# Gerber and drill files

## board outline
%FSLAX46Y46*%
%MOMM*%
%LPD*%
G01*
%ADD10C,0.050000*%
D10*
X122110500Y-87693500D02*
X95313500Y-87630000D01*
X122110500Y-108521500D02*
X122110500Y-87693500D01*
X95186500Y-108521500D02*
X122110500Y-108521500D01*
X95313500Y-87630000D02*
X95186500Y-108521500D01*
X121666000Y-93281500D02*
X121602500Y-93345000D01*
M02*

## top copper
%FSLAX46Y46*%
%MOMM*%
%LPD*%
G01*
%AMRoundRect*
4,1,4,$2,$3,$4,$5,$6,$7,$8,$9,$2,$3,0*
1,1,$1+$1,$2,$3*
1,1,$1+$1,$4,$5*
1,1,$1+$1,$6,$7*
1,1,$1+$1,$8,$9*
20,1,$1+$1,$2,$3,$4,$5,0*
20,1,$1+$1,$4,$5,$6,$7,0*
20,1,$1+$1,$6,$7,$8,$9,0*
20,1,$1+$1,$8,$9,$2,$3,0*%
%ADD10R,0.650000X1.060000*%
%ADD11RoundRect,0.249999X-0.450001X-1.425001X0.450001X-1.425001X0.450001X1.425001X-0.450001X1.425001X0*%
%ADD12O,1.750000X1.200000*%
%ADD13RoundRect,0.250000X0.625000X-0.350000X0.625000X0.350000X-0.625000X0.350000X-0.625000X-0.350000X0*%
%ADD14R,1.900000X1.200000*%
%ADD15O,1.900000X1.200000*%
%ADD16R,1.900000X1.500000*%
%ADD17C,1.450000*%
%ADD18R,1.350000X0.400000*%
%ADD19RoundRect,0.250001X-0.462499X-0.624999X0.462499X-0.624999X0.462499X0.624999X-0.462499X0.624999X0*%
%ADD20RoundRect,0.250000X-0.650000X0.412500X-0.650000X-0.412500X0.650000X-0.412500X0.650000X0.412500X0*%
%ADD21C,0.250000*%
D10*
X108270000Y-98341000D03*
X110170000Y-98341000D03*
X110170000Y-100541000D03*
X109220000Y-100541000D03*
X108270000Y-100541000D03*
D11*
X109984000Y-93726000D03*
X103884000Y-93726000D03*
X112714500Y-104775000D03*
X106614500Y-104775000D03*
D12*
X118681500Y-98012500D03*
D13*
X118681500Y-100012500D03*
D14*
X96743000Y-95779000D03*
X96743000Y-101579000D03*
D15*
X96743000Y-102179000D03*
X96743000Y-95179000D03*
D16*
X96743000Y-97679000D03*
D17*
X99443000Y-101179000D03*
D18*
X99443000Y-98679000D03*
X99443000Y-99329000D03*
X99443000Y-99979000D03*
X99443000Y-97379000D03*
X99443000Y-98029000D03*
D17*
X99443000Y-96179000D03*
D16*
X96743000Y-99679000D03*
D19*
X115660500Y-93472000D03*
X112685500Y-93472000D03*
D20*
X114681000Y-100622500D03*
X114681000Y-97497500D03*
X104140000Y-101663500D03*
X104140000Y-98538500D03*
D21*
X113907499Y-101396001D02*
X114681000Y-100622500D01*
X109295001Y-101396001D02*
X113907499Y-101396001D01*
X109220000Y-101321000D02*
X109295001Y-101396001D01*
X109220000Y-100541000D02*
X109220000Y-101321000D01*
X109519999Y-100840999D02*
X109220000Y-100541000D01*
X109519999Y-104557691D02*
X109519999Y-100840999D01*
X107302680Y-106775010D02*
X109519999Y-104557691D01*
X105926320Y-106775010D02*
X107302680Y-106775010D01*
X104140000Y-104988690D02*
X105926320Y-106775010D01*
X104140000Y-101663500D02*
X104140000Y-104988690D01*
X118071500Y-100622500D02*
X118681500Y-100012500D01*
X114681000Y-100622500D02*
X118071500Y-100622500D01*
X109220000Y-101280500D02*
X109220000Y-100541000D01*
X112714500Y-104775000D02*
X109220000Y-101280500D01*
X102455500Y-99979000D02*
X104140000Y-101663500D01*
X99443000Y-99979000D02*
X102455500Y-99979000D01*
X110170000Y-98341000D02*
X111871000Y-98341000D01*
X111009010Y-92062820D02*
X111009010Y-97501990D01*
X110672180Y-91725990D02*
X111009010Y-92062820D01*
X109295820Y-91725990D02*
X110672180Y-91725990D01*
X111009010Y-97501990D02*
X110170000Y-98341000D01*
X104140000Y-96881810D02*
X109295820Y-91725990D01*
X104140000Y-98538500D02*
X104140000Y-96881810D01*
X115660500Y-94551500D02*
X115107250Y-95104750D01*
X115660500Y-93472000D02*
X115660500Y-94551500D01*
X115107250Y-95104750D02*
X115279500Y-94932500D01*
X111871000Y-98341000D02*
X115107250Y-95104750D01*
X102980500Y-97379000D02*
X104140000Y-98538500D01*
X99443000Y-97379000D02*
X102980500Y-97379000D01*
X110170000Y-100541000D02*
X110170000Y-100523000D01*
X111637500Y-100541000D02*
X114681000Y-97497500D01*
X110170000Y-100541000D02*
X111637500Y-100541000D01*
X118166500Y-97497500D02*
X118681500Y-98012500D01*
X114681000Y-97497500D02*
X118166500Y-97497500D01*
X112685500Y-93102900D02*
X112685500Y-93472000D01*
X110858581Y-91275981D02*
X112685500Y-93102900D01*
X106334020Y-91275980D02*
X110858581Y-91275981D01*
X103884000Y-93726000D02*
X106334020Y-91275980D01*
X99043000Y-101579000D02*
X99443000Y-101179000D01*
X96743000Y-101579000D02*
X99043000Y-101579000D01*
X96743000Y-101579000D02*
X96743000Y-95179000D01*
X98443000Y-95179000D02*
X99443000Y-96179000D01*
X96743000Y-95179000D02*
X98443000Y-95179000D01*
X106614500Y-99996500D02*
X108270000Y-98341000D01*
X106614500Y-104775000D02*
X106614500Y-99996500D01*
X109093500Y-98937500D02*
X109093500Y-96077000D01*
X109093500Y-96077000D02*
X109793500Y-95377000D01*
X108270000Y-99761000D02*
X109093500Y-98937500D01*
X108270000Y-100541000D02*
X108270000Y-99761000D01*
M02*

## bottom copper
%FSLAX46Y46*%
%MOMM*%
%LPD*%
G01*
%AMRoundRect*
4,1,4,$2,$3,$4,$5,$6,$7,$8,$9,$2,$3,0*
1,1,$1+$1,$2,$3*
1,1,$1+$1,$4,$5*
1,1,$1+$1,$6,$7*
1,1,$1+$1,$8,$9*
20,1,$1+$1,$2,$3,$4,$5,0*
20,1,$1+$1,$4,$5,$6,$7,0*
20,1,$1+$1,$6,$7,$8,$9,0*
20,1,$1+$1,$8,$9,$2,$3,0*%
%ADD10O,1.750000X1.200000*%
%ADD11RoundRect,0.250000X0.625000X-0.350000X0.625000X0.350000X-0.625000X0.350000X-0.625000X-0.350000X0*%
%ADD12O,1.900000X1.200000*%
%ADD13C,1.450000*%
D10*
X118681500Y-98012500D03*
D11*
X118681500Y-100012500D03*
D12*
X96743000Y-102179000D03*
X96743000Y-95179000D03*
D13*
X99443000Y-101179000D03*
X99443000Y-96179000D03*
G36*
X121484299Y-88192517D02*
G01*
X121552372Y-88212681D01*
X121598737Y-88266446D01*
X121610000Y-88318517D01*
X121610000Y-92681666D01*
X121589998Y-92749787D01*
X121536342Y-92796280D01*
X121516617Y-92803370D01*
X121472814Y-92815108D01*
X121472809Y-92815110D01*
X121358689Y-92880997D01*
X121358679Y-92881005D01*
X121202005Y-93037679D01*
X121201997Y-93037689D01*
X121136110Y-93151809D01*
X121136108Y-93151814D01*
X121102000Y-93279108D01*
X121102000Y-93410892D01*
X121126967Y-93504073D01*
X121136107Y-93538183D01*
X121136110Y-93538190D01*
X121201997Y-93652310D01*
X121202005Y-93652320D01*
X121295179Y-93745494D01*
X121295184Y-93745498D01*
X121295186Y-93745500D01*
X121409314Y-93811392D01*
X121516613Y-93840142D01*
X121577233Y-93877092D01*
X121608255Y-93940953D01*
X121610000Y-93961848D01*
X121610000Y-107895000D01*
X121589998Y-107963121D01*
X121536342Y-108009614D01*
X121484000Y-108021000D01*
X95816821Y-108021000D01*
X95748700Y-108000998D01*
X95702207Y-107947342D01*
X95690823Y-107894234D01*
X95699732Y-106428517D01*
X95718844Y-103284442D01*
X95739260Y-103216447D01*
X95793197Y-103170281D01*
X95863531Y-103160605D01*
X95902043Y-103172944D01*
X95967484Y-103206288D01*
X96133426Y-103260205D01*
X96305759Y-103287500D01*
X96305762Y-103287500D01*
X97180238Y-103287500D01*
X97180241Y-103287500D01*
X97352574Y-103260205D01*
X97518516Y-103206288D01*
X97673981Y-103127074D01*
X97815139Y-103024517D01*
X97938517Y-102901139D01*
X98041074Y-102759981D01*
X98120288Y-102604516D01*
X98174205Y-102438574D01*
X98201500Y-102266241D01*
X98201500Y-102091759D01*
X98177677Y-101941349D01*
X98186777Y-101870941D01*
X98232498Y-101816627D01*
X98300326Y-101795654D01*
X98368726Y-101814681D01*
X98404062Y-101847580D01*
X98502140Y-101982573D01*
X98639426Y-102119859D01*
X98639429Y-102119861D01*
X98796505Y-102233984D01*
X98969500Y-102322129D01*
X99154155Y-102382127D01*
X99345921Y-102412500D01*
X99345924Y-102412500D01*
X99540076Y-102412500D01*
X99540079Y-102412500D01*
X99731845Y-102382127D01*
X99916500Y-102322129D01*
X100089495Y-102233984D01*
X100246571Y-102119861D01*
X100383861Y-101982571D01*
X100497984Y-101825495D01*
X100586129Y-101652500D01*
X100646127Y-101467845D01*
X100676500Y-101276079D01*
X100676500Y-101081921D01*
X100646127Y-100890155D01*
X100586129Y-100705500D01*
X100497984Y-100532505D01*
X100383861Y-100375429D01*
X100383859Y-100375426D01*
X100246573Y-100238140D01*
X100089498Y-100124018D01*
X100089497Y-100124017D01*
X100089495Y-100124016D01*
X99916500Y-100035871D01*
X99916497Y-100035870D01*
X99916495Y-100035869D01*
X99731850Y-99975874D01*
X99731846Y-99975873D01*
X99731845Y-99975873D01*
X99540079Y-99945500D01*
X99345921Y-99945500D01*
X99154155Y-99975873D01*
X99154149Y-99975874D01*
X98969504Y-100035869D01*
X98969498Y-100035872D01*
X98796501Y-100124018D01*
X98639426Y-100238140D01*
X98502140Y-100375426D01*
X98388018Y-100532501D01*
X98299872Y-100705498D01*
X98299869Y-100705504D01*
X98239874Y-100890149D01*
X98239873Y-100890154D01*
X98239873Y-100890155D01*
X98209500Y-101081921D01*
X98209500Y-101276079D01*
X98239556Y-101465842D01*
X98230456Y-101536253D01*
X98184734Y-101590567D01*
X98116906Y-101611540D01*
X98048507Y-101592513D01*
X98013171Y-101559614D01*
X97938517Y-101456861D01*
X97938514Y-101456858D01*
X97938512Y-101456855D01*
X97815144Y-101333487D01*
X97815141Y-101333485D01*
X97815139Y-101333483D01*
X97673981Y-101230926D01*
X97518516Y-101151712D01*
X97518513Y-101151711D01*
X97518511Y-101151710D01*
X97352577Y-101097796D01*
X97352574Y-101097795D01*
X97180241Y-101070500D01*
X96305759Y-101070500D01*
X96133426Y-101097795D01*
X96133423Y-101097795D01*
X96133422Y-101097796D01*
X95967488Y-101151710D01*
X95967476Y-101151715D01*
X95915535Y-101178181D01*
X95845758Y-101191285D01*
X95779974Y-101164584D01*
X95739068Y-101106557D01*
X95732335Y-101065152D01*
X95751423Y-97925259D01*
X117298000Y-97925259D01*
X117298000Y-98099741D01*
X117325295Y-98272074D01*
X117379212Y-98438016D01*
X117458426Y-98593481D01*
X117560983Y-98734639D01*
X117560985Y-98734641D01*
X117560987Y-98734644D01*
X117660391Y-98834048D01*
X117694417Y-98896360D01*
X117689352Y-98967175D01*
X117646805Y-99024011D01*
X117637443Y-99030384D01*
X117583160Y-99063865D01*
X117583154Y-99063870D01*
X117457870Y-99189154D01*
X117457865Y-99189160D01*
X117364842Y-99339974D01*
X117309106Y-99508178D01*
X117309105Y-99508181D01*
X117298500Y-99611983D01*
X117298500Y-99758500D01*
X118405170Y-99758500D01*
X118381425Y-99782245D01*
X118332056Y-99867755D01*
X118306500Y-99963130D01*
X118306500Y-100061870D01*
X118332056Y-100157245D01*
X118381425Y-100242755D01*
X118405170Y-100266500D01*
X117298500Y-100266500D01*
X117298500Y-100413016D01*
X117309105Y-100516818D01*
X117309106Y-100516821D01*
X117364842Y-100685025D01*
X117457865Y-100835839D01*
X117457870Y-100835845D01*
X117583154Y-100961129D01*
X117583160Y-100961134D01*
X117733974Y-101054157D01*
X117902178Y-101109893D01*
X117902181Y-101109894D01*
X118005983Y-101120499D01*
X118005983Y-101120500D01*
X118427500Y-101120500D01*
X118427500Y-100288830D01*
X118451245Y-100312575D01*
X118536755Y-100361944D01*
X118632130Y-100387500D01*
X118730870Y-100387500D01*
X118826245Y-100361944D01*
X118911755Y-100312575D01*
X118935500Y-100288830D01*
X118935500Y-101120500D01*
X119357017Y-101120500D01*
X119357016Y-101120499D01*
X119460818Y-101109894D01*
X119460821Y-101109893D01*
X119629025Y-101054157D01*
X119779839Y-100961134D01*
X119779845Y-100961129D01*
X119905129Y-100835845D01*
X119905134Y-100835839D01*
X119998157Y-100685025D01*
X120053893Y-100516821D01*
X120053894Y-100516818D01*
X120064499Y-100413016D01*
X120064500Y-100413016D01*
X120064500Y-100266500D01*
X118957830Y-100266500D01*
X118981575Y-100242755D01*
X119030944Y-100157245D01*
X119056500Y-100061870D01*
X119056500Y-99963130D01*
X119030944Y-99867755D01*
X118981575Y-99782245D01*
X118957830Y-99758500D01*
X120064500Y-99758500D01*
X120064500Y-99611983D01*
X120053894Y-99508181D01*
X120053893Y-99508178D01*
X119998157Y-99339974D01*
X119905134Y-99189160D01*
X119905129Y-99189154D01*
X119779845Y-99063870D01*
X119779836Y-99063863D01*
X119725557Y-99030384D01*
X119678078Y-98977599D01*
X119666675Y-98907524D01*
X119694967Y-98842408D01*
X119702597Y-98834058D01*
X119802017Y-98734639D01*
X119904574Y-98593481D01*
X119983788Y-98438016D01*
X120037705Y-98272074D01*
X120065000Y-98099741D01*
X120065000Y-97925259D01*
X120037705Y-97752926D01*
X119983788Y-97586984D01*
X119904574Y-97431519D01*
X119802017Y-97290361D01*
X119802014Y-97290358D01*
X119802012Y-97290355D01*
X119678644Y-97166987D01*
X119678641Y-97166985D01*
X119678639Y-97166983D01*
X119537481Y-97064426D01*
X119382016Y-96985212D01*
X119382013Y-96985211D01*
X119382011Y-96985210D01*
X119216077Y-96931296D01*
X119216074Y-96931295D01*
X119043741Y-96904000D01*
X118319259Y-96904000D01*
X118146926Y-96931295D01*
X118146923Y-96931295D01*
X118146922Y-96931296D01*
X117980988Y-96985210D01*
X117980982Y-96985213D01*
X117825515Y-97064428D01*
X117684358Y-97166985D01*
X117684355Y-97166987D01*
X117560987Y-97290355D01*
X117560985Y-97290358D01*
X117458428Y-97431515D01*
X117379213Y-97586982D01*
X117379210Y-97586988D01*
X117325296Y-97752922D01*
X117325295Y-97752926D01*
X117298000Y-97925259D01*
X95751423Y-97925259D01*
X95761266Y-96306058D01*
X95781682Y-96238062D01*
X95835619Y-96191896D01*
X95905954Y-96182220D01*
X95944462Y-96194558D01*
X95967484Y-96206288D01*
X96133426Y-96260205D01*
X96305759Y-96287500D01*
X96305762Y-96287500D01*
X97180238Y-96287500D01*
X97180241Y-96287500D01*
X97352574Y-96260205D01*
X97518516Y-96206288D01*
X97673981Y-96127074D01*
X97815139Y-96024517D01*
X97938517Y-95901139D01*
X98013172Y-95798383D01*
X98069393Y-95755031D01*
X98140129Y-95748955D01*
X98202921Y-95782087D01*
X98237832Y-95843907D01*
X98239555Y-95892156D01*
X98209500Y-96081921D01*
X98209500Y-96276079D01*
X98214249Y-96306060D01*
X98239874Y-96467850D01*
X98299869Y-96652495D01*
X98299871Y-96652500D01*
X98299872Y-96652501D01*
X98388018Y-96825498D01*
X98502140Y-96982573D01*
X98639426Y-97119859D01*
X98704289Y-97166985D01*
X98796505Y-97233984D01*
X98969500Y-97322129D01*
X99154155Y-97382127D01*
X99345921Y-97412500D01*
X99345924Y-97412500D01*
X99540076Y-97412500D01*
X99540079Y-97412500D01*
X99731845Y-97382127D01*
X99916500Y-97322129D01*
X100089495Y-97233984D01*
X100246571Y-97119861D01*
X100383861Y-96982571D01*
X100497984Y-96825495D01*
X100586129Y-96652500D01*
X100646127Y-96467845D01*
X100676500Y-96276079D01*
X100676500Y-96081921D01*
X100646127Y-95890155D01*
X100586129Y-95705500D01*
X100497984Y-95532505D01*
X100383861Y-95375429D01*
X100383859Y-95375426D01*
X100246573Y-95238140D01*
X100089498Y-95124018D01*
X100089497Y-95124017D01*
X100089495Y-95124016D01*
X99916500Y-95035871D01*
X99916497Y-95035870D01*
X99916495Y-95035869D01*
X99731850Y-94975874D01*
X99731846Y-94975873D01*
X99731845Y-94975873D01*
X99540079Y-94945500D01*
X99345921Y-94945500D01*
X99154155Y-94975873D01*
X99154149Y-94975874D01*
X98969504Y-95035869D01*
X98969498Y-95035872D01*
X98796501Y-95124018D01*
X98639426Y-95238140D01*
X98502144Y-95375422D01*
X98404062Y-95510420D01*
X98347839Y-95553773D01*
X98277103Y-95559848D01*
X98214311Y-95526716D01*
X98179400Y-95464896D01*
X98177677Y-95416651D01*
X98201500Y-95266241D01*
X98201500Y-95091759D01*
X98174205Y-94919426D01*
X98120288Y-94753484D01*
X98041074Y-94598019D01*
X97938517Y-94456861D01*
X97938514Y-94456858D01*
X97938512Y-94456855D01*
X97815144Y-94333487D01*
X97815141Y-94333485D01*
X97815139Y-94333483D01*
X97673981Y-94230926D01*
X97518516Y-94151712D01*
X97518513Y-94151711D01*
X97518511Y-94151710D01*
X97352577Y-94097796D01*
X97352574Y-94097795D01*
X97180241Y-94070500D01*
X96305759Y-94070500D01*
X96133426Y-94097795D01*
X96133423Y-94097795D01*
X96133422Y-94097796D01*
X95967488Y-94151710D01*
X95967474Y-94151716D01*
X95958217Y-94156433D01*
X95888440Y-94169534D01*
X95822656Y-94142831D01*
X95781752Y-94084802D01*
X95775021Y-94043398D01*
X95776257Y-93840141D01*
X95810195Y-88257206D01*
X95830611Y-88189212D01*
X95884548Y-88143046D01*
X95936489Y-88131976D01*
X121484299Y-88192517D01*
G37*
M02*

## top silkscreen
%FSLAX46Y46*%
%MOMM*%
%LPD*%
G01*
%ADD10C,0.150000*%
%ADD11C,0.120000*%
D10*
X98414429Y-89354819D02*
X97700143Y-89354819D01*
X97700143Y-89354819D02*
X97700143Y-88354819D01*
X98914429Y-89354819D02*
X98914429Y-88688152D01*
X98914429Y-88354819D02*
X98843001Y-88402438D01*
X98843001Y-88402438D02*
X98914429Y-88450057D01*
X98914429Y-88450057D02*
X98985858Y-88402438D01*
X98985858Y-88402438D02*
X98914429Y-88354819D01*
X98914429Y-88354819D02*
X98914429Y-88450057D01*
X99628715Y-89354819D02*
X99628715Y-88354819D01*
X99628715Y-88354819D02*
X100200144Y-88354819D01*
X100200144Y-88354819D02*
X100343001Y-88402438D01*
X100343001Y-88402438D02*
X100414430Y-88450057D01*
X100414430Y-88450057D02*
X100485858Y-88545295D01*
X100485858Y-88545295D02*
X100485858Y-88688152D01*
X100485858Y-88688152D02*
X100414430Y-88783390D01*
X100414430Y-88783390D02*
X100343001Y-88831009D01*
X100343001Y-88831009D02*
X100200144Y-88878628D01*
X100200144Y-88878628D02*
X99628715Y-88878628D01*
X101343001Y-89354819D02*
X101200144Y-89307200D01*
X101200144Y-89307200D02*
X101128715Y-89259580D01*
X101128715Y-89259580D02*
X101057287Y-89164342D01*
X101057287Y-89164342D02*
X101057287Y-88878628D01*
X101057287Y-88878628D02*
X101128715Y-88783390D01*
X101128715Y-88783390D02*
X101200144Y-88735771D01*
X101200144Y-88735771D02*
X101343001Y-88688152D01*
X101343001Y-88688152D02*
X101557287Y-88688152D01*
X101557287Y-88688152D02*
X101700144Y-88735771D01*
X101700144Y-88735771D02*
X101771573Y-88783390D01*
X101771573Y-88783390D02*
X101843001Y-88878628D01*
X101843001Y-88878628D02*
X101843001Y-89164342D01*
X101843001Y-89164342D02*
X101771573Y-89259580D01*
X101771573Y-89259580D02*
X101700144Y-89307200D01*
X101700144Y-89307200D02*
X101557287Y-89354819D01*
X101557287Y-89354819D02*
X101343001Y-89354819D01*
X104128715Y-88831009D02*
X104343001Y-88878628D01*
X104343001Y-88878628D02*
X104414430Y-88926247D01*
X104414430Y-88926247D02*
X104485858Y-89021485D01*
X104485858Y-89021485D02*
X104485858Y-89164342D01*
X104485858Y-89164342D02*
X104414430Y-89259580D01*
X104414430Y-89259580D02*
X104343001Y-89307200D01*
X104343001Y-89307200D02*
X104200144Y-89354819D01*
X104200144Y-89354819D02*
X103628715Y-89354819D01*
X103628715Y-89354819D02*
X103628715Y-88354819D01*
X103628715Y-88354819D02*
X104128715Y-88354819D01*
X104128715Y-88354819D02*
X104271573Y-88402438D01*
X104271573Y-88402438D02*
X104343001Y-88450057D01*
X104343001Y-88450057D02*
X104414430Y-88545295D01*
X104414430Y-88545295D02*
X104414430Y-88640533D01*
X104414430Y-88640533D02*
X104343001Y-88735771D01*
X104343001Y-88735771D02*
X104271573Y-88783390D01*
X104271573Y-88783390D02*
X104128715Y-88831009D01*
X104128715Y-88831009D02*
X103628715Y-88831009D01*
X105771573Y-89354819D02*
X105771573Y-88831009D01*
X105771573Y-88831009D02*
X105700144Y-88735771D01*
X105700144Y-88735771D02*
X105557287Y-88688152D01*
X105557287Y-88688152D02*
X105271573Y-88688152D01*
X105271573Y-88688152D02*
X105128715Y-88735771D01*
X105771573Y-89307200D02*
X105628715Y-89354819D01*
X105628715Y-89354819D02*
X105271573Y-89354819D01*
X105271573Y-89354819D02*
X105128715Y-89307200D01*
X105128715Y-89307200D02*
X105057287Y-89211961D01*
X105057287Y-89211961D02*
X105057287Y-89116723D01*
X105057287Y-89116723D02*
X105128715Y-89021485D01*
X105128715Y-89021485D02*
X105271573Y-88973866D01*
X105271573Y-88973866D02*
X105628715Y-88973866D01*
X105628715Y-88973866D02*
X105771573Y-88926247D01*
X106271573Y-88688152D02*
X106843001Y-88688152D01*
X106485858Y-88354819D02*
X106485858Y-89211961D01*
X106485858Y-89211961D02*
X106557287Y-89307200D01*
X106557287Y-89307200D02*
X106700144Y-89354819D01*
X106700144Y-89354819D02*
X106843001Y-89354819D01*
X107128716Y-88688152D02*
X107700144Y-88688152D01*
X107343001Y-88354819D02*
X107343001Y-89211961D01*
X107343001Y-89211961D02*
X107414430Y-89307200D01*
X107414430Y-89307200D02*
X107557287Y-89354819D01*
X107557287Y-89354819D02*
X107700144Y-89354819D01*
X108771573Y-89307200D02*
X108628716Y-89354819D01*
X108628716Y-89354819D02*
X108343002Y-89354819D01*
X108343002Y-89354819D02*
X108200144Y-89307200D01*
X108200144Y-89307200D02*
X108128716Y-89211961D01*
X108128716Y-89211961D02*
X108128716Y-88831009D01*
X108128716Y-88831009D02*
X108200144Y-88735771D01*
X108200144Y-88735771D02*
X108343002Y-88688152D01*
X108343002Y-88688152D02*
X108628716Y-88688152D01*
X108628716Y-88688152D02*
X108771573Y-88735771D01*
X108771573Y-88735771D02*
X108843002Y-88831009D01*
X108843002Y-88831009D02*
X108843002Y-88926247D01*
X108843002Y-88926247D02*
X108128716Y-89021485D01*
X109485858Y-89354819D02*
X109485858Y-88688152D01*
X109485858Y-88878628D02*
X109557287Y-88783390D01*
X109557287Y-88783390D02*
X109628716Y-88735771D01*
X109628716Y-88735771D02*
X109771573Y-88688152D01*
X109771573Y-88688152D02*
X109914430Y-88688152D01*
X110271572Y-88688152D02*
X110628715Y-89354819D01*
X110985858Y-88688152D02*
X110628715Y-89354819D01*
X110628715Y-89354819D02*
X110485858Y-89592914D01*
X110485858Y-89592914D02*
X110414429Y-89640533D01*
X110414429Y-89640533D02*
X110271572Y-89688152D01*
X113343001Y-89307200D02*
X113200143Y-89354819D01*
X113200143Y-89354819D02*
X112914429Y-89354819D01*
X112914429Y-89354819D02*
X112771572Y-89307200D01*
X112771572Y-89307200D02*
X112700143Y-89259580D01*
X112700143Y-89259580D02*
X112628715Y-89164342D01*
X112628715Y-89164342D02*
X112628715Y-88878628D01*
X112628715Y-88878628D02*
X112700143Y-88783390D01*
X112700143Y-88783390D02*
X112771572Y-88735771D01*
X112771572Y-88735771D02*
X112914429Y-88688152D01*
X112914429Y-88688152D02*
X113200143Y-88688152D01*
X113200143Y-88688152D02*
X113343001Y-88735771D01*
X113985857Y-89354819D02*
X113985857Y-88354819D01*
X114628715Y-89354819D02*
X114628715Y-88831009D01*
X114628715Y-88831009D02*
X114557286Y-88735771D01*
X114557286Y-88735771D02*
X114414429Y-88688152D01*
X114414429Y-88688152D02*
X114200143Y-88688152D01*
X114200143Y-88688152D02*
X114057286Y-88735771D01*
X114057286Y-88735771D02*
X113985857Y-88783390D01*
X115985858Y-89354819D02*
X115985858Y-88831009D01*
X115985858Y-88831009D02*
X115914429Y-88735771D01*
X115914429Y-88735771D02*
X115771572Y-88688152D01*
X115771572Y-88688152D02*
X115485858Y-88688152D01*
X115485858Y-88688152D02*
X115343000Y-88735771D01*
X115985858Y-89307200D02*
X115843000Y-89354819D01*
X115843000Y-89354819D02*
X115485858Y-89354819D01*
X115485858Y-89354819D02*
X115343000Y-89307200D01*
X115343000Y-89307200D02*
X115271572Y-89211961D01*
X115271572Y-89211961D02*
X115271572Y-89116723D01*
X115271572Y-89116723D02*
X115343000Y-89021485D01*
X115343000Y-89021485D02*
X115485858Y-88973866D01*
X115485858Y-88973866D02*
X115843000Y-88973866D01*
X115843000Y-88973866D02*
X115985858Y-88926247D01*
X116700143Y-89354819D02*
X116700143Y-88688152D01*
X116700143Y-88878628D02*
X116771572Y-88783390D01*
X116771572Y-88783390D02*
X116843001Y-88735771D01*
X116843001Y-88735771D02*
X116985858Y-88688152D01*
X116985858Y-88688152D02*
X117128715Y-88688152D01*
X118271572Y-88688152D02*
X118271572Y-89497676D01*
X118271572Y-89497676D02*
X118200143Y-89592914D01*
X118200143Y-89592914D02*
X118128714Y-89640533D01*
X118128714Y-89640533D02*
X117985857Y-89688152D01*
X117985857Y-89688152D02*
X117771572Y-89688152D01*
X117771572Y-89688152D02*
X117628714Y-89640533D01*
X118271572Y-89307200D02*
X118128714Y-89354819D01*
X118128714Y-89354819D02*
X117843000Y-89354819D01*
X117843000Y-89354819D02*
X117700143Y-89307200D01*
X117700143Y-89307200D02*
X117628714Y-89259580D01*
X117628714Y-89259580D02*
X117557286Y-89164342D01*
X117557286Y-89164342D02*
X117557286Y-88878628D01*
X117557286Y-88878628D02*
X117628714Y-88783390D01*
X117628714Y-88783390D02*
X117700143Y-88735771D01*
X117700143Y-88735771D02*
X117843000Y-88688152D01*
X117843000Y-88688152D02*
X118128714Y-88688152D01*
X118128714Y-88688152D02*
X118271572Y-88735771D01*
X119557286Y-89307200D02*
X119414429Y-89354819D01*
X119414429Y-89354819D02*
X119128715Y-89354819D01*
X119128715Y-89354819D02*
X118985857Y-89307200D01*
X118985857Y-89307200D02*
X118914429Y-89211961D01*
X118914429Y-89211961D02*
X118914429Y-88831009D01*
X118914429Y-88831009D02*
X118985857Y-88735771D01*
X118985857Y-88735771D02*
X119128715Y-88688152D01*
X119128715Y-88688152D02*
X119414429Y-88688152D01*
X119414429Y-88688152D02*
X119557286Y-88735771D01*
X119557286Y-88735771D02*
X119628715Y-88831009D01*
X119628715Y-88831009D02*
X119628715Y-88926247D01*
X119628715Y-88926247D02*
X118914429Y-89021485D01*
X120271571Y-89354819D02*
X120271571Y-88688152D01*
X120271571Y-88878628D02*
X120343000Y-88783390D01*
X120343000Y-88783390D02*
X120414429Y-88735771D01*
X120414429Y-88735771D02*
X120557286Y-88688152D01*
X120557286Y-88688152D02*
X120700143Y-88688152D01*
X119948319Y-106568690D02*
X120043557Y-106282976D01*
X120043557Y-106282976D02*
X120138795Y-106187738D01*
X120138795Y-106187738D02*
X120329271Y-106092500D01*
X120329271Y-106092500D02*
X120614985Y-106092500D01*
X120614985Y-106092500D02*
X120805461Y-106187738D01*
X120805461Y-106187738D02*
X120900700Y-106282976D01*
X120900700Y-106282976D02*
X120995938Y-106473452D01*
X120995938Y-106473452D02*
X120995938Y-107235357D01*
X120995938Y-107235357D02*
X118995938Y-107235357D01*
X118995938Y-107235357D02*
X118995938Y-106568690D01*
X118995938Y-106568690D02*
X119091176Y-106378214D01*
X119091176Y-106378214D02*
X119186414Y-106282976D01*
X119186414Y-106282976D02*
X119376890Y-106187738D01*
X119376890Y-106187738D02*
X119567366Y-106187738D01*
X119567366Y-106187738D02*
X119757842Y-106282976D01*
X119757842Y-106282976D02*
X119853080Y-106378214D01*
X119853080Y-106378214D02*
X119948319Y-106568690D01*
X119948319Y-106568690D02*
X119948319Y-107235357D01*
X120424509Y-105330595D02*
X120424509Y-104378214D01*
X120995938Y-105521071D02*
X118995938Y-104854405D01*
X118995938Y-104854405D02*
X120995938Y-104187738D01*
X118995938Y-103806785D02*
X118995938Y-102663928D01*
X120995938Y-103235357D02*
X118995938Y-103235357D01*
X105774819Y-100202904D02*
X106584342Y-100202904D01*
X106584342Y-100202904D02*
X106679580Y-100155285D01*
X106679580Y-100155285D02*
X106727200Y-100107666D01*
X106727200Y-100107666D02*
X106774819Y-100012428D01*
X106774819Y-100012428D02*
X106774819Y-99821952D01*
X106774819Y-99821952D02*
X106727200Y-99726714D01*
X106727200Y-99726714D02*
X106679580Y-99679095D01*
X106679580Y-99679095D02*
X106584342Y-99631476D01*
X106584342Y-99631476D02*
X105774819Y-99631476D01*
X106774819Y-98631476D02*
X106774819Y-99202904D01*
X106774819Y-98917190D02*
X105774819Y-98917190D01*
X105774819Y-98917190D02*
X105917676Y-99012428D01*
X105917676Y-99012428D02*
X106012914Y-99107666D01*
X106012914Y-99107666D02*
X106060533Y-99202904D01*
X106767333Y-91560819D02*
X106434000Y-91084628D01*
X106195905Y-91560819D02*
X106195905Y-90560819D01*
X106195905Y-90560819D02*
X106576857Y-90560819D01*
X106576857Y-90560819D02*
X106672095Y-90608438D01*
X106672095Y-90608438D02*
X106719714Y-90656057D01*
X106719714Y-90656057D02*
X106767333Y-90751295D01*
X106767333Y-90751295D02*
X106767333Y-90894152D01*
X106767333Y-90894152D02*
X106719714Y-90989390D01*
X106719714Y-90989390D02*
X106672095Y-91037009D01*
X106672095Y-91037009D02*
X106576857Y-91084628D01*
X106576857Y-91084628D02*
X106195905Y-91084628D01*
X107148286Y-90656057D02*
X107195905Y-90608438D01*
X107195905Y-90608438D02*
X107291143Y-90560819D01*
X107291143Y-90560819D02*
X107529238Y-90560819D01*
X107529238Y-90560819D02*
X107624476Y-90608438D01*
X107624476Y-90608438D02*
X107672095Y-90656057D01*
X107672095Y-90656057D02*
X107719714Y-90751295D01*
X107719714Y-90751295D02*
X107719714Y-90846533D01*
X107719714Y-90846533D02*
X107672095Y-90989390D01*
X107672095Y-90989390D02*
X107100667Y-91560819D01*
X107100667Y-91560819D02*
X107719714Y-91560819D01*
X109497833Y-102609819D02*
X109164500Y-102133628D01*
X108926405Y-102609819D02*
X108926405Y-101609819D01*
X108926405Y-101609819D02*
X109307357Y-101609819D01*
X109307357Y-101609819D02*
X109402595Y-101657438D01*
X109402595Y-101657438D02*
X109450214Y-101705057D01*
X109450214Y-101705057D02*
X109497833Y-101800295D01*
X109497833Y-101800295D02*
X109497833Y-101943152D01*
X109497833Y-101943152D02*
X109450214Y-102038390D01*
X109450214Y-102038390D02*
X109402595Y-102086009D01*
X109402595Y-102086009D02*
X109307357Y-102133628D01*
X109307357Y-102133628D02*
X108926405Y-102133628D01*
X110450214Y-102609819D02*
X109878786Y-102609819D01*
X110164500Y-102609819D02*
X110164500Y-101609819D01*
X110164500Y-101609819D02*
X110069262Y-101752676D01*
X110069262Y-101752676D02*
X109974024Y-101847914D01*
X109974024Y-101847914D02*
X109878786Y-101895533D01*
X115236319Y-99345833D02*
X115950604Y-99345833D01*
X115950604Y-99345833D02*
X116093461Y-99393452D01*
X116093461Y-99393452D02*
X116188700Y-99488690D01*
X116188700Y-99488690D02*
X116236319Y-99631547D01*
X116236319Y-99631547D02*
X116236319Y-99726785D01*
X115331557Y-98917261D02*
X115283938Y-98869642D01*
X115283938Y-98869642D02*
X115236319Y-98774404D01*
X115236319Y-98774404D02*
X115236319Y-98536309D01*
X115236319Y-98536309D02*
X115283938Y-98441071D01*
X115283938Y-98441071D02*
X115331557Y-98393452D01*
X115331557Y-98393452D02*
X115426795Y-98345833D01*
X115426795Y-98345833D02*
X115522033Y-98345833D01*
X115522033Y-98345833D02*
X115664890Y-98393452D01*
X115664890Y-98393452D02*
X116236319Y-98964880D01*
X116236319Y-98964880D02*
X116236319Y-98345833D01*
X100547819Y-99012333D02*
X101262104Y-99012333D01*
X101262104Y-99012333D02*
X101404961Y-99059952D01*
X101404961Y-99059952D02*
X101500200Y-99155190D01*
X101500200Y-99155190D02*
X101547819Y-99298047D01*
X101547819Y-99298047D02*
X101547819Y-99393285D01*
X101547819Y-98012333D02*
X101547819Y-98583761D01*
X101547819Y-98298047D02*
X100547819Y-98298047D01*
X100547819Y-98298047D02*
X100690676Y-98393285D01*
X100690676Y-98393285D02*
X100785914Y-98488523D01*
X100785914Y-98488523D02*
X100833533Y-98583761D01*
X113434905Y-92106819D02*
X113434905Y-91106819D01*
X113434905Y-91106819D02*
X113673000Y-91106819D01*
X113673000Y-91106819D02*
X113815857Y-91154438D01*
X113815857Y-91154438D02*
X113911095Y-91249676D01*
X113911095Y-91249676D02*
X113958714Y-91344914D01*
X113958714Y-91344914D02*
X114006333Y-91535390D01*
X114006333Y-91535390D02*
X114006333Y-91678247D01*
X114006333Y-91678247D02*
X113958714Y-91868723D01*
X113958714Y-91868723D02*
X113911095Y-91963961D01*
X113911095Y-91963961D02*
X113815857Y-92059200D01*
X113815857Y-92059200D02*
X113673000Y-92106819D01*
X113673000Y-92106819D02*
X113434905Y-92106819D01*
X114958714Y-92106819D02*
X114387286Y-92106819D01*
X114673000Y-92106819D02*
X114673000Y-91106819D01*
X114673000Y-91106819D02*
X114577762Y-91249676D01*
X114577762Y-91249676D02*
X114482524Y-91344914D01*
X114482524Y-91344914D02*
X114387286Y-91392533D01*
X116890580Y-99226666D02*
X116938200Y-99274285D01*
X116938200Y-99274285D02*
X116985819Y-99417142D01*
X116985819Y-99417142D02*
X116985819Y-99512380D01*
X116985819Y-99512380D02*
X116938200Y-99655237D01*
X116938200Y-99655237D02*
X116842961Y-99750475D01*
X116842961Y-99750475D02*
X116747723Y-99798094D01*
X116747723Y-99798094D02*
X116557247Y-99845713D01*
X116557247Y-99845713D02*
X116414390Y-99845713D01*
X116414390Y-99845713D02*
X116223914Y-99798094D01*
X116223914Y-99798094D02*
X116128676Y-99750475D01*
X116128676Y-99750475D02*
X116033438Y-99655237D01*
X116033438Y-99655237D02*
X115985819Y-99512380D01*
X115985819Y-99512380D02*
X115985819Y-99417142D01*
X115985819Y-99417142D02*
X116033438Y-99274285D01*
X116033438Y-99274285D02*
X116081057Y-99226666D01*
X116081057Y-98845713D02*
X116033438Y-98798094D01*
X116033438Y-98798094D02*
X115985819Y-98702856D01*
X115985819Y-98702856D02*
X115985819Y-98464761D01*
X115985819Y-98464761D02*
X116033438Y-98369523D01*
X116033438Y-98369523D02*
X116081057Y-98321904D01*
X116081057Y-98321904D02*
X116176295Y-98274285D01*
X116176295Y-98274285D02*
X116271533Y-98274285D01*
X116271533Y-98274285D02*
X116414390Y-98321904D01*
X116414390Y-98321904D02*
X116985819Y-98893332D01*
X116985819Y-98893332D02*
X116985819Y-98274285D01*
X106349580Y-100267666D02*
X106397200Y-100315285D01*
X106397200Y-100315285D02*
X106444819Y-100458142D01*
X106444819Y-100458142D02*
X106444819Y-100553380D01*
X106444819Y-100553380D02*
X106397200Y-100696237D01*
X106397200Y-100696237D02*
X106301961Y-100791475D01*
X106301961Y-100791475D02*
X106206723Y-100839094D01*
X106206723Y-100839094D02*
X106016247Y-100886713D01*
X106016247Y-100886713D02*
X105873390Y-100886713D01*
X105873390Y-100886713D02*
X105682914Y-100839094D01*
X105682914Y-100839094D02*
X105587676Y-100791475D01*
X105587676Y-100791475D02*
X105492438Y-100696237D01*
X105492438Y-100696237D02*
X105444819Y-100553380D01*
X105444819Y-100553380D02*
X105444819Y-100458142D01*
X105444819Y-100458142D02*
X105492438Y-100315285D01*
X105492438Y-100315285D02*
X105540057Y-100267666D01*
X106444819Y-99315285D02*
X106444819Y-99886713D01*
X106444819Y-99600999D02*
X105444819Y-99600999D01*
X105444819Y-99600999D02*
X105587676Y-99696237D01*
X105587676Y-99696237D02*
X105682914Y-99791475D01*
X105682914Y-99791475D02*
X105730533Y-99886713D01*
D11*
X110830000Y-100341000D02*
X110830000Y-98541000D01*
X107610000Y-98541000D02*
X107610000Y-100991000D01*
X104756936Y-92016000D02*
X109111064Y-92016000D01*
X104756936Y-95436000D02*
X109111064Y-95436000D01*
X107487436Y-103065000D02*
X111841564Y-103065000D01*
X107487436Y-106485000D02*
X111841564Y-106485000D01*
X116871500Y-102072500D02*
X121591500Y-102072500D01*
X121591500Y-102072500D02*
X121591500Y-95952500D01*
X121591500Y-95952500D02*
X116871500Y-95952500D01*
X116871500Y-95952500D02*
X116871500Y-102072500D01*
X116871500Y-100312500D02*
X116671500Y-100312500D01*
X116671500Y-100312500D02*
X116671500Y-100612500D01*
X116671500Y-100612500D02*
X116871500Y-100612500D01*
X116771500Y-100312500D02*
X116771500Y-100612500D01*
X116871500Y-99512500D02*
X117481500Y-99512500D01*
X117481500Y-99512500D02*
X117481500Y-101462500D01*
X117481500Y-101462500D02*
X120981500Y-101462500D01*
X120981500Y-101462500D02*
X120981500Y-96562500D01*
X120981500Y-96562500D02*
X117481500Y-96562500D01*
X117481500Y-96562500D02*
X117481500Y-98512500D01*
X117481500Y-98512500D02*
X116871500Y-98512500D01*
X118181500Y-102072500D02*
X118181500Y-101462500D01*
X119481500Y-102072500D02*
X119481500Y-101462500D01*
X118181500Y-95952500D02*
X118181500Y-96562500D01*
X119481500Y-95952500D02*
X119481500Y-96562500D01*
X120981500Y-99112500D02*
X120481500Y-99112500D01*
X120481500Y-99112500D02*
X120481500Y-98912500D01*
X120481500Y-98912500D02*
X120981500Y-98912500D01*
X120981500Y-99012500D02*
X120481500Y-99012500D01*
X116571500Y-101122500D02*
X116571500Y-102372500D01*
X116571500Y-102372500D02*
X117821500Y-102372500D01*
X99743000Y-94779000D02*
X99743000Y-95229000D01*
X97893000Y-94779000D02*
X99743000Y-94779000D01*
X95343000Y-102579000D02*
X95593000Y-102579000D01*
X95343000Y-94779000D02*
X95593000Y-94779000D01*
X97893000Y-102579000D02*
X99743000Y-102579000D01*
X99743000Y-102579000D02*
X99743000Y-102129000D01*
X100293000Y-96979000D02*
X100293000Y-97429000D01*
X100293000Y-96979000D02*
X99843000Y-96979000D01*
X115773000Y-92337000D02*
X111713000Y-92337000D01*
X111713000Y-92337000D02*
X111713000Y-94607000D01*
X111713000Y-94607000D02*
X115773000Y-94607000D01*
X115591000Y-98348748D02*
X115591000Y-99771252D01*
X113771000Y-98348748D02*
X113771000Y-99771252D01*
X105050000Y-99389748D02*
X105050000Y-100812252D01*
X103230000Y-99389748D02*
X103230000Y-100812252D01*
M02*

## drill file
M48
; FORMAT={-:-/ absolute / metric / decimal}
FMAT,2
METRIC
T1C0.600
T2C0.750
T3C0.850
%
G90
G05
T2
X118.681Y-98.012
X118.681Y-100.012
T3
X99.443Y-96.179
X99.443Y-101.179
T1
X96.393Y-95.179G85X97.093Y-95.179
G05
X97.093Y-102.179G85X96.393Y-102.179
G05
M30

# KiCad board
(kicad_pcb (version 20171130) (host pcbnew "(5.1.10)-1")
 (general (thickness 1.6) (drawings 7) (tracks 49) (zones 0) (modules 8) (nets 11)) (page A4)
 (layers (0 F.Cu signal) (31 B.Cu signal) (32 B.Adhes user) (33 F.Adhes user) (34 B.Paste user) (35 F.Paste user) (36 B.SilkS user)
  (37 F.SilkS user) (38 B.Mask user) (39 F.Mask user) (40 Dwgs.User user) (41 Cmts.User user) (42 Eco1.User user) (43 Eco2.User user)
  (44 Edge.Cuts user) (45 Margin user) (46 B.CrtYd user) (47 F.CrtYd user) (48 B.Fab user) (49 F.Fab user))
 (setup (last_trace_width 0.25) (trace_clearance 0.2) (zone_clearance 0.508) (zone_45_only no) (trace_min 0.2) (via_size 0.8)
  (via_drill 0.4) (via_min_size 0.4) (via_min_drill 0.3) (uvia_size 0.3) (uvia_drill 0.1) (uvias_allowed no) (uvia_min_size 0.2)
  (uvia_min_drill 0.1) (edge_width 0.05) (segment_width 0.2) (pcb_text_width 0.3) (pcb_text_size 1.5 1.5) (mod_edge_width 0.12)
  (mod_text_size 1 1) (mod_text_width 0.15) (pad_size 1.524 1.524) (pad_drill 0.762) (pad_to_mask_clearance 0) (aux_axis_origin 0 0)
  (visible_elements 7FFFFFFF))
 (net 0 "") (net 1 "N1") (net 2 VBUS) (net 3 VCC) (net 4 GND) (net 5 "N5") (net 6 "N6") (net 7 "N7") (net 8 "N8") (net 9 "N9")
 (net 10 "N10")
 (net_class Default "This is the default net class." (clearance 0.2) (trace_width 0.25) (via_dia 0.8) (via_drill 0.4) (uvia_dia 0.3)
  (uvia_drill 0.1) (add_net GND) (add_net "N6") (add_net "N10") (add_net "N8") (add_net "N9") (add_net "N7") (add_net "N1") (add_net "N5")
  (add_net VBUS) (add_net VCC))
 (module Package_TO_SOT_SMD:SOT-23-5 (layer F.Cu) (at 109.22 99.441 90)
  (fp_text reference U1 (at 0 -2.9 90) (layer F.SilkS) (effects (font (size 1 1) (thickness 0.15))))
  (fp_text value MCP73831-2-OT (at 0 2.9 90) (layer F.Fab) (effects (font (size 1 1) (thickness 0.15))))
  (fp_line (start -0.9 1.61) (end 0.9 1.61) (layer F.SilkS) (width 0.12))
  (fp_line (start 0.9 -1.61) (end -1.55 -1.61) (layer F.SilkS) (width 0.12))
  (pad 5 smd rect (at 1.1 -0.95 90) (size 1.06 0.65) (layers F.Cu F.Paste F.Mask) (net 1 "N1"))
  (pad 4 smd rect (at 1.1 0.95 90) (size 1.06 0.65) (layers F.Cu F.Paste F.Mask) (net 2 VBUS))
  (pad 3 smd rect (at -1.1 0.95 90) (size 1.06 0.65) (layers F.Cu F.Paste F.Mask) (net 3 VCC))
  (pad 2 smd rect (at -1.1 0 90) (size 1.06 0.65) (layers F.Cu F.Paste F.Mask) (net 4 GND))
  (pad 1 smd rect (at -1.1 -0.95 90) (size 1.06 0.65) (layers F.Cu F.Paste F.Mask) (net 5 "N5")))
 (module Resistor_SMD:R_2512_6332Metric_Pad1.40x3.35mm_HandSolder (layer F.Cu) (at 106.934 93.726)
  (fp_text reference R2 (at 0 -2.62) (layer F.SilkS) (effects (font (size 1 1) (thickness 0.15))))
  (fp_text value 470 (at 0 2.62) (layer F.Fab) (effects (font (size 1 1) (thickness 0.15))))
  (fp_line (start -2.177064 -1.71) (end 2.177064 -1.71) (layer F.SilkS) (width 0.12))
  (fp_line (start -2.177064 1.71) (end 2.177064 1.71) (layer F.SilkS) (width 0.12))
  (pad 2 smd roundrect (at 3.05 0) (size 1.4 3.35) (layers F.Cu F.Paste F.Mask) (roundrect_rratio 0.178571) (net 5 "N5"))
  (pad 1 smd roundrect (at -3.05 0) (size 1.4 3.35) (layers F.Cu F.Paste F.Mask) (roundrect_rratio 0.178571) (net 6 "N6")))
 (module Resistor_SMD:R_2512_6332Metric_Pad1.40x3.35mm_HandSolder (layer F.Cu) (at 109.6645 104.775)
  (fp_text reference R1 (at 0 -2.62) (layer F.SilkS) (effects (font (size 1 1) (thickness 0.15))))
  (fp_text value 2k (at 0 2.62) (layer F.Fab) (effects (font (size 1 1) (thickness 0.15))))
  (fp_line (start -2.177064 -1.71) (end 2.177064 -1.71) (layer F.SilkS) (width 0.12))
  (fp_line (start -2.177064 1.71) (end 2.177064 1.71) (layer F.SilkS) (width 0.12))
  (pad 2 smd roundrect (at 3.05 0) (size 1.4 3.35) (layers F.Cu F.Paste F.Mask) (roundrect_rratio 0.178571) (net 4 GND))
  (pad 1 smd roundrect (at -3.05 0) (size 1.4 3.35) (layers F.Cu F.Paste F.Mask) (roundrect_rratio 0.178571) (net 1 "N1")))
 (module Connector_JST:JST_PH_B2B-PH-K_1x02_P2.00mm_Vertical (layer F.Cu) (at 118.6815 100.0125 90)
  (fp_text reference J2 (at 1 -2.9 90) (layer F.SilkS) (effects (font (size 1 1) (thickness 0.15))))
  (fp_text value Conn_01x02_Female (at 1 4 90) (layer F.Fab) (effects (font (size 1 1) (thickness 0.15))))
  (fp_line (start -2.06 -1.81) (end -2.06 2.91) (layer F.SilkS) (width 0.12))
  (fp_line (start -2.06 2.91) (end 4.06 2.91) (layer F.SilkS) (width 0.12))
  (fp_line (start 4.06 2.91) (end 4.06 -1.81) (layer F.SilkS) (width 0.12))
  (fp_line (start 4.06 -1.81) (end -2.06 -1.81) (layer F.SilkS) (width 0.12))
  (fp_line (start -0.3 -1.81) (end -0.3 -2.01) (layer F.SilkS) (width 0.12))
  (fp_line (start -0.3 -2.01) (end -0.6 -2.01) (layer F.SilkS) (width 0.12))
  (fp_line (start -0.6 -2.01) (end -0.6 -1.81) (layer F.SilkS) (width 0.12))
  (fp_line (start -0.3 -1.91) (end -0.6 -1.91) (layer F.SilkS) (width 0.12))
  (fp_line (start 0.5 -1.81) (end 0.5 -1.2) (layer F.SilkS) (width 0.12))
  (fp_line (start 0.5 -1.2) (end -1.45 -1.2) (layer F.SilkS) (width 0.12))
  (fp_line (start -1.45 -1.2) (end -1.45 2.3) (layer F.SilkS) (width 0.12))
  (fp_line (start -1.45 2.3) (end 3.45 2.3) (layer F.SilkS) (width 0.12))
  (fp_line (start 3.45 2.3) (end 3.45 -1.2) (layer F.SilkS) (width 0.12))
  (fp_line (start 3.45 -1.2) (end 1.5 -1.2) (layer F.SilkS) (width 0.12))
  (fp_line (start 1.5 -1.2) (end 1.5 -1.81) (layer F.SilkS) (width 0.12))
  (fp_line (start -2.06 -0.5) (end -1.45 -0.5) (layer F.SilkS) (width 0.12))
  (fp_line (start -2.06 0.8) (end -1.45 0.8) (layer F.SilkS) (width 0.12))
  (fp_line (start 4.06 -0.5) (end 3.45 -0.5) (layer F.SilkS) (width 0.12))
  (fp_line (start 4.06 0.8) (end 3.45 0.8) (layer F.SilkS) (width 0.12))
  (fp_line (start 0.9 2.3) (end 0.9 1.8) (layer F.SilkS) (width 0.12))
  (fp_line (start 0.9 1.8) (end 1.1 1.8) (layer F.SilkS) (width 0.12))
  (fp_line (start 1.1 1.8) (end 1.1 2.3) (layer F.SilkS) (width 0.12))
  (fp_line (start 1 2.3) (end 1 1.8) (layer F.SilkS) (width 0.12))
  (fp_line (start -1.11 -2.11) (end -2.36 -2.11) (layer F.SilkS) (width 0.12))
  (fp_line (start -2.36 -2.11) (end -2.36 -0.86) (layer F.SilkS) (width 0.12))
  (pad 2 thru_hole oval (at 2 0 90) (size 1.2 1.75) (drill 0.75) (layers *.Cu *.Mask) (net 3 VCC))
  (pad 1 thru_hole roundrect (at 0 0 90) (size 1.2 1.75) (drill 0.75) (layers *.Cu *.Mask) (roundrect_rratio 0.208333) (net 4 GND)))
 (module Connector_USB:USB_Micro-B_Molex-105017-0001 (layer F.Cu) (at 97.9805 98.679 270)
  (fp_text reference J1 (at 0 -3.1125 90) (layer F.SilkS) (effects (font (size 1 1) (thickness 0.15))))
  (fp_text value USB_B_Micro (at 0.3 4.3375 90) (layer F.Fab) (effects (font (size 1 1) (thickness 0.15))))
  (fp_line (start -3.9 -1.7625) (end -3.45 -1.7625) (layer F.SilkS) (width 0.12))
  (fp_line (start -3.9 0.0875) (end -3.9 -1.7625) (layer F.SilkS) (width 0.12))
  (fp_line (start 3.9 2.6375) (end 3.9 2.3875) (layer F.SilkS) (width 0.12))
  (fp_line (start -3.9 2.6375) (end -3.9 2.3875) (layer F.SilkS) (width 0.12))
  (fp_line (start 3.9 0.0875) (end 3.9 -1.7625) (layer F.SilkS) (width 0.12))
  (fp_line (start 3.9 -1.7625) (end 3.45 -1.7625) (layer F.SilkS) (width 0.12))
  (fp_line (start -1.7 -2.3125) (end -1.25 -2.3125) (layer F.SilkS) (width 0.12))
  (fp_line (start -1.7 -2.3125) (end -1.7 -1.8625) (layer F.SilkS) (width 0.12))
  (pad 6 smd rect (at -2.9 1.2375 270) (size 1.2 1.9) (layers F.Cu F.Mask) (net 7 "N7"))
  (pad 6 smd rect (at 2.9 1.2375 270) (size 1.2 1.9) (layers F.Cu F.Mask) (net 7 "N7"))
  (pad 6 thru_hole oval (at 3.5 1.2375 270) (size 1.2 1.9) (drill oval 0.6 1.3) (layers *.Cu *.Mask) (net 7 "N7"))
  (pad 6 thru_hole oval (at -3.5 1.2375 90) (size 1.2 1.9) (drill oval 0.6 1.3) (layers *.Cu *.Mask) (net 7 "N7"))
  (pad 6 smd rect (at -1 1.2375 270) (size 1.5 1.9) (layers F.Cu F.Paste F.Mask) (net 7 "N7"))
  (pad 6 thru_hole circle (at 2.5 -1.4625 270) (size 1.45 1.45) (drill 0.85) (layers *.Cu *.Mask) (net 7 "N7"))
  (pad 3 smd rect (at 0 -1.4625 270) (size 0.4 1.35) (layers F.Cu F.Paste F.Mask) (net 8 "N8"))
  (pad 4 smd rect (at 0.65 -1.4625 270) (size 0.4 1.35) (layers F.Cu F.Paste F.Mask) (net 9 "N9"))
  (pad 5 smd rect (at 1.3 -1.4625 270) (size 0.4 1.35) (layers F.Cu F.Paste F.Mask) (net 4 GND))
  (pad 1 smd rect (at -1.3 -1.4625 270) (size 0.4 1.35) (layers F.Cu F.Paste F.Mask) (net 2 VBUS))
  (pad 2 smd rect (at -0.65 -1.4625 270) (size 0.4 1.35) (layers F.Cu F.Paste F.Mask) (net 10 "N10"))
  (pad 6 thru_hole circle (at -2.5 -1.4625 270) (size 1.45 1.45) (drill 0.85) (layers *.Cu *.Mask) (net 7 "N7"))
  (pad 6 smd rect (at 1 1.2375 270) (size 1.5 1.9) (layers F.Cu F.Paste F.Mask) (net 7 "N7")))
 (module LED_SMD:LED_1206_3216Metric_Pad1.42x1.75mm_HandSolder (layer F.Cu) (at 114.173 93.472)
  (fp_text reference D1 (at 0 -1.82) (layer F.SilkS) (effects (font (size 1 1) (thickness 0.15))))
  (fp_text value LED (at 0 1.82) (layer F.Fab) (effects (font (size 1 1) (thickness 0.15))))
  (fp_line (start 1.6 -1.135) (end -2.46 -1.135) (layer F.SilkS) (width 0.12))
  (fp_line (start -2.46 -1.135) (end -2.46 1.135) (layer F.SilkS) (width 0.12))
  (fp_line (start -2.46 1.135) (end 1.6 1.135) (layer F.SilkS) (width 0.12))
  (pad 2 smd roundrect (at 1.4875 0) (size 1.425 1.75) (layers F.Cu F.Paste F.Mask) (roundrect_rratio 0.175439) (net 2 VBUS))
  (pad 1 smd roundrect (at -1.4875 0) (size 1.425 1.75) (layers F.Cu F.Paste F.Mask) (roundrect_rratio 0.175439) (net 6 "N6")))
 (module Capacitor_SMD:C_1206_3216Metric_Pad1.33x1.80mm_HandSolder (layer F.Cu) (at 114.681 99.06 270)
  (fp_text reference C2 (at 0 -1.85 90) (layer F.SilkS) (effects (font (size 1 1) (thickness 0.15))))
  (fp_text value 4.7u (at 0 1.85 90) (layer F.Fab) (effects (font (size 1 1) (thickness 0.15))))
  (fp_line (start -0.711252 -0.91) (end 0.711252 -0.91) (layer F.SilkS) (width 0.12))
  (fp_line (start -0.711252 0.91) (end 0.711252 0.91) (layer F.SilkS) (width 0.12))
  (pad 2 smd roundrect (at 1.5625 0 270) (size 1.325 1.8) (layers F.Cu F.Paste F.Mask) (roundrect_rratio 0.188679) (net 4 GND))
  (pad 1 smd roundrect (at -1.5625 0 270) (size 1.325 1.8) (layers F.Cu F.Paste F.Mask) (roundrect_rratio 0.188679) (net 3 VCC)))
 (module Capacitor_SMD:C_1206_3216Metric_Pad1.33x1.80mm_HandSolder (layer F.Cu) (at 104.14 100.101 270)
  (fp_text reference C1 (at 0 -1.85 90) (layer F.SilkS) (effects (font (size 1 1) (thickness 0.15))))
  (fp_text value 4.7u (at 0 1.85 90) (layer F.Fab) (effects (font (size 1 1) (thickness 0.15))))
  (fp_line (start -0.711252 -0.91) (end 0.711252 -0.91) (layer F.SilkS) (width 0.12))
  (fp_line (start -0.711252 0.91) (end 0.711252 0.91) (layer F.SilkS) (width 0.12))
  (pad 2 smd roundrect (at 1.5625 0 270) (size 1.325 1.8) (layers F.Cu F.Paste F.Mask) (roundrect_rratio 0.188679) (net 4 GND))
  (pad 1 smd roundrect (at -1.5625 0 270) (size 1.325 1.8) (layers F.Cu F.Paste F.Mask) (roundrect_rratio 0.188679) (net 2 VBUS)))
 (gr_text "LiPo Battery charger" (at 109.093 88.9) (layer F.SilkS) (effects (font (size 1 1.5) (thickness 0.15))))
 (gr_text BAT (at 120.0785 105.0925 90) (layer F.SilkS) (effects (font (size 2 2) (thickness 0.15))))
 (gr_line (start 122.1105 87.6935) (end 95.3135 87.63) (layer Edge.Cuts) (width 0.05))
 (gr_line (start 122.1105 108.5215) (end 122.1105 87.6935) (layer Edge.Cuts) (width 0.05))
 (gr_line (start 95.1865 108.5215) (end 122.1105 108.5215) (layer Edge.Cuts) (width 0.05))
 (gr_line (start 95.3135 87.63) (end 95.1865 108.5215) (layer Edge.Cuts) (width 0.05))
 (gr_line (start 121.666 93.2815) (end 121.6025 93.345) (layer Edge.Cuts) (width 0.05))
 (segment (start 113.907499 101.396001) (end 114.681 100.6225) (width 0.25) (layer F.Cu) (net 4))
 (segment (start 109.295001 101.396001) (end 113.907499 101.396001) (width 0.25) (layer F.Cu) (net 4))
 (segment (start 109.22 101.321) (end 109.295001 101.396001) (width 0.25) (layer F.Cu) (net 4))
 (segment (start 109.22 100.541) (end 109.22 101.321) (width 0.25) (layer F.Cu) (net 4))
 (segment (start 109.519999 100.840999) (end 109.22 100.541) (width 0.25) (layer F.Cu) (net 4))
 (segment (start 109.519999 104.557691) (end 109.519999 100.840999) (width 0.25) (layer F.Cu) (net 4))
 (segment (start 107.30268 106.77501) (end 109.519999 104.557691) (width 0.25) (layer F.Cu) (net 4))
 (segment (start 105.92632 106.77501) (end 107.30268 106.77501) (width 0.25) (layer F.Cu) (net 4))
 (segment (start 104.14 104.98869) (end 105.92632 106.77501) (width 0.25) (layer F.Cu) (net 4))
 (segment (start 104.14 101.6635) (end 104.14 104.98869) (width 0.25) (layer F.Cu) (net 4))
 (segment (start 118.0715 100.6225) (end 118.6815 100.0125) (width 0.25) (layer F.Cu) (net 4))
 (segment (start 114.681 100.6225) (end 118.0715 100.6225) (width 0.25) (layer F.Cu) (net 4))
 (segment (start 109.22 101.2805) (end 109.22 100.541) (width 0.25) (layer F.Cu) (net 4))
 (segment (start 112.7145 104.775) (end 109.22 101.2805) (width 0.25) (layer F.Cu) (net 4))
 (segment (start 102.4555 99.979) (end 104.14 101.6635) (width 0.25) (layer F.Cu) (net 4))
 (segment (start 99.443 99.979) (end 102.4555 99.979) (width 0.25) (layer F.Cu) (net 4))
 (segment (start 110.17 98.341) (end 111.871 98.341) (width 0.25) (layer F.Cu) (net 2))
 (segment (start 111.00901 92.06282) (end 111.00901 97.50199) (width 0.25) (layer F.Cu) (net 2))
 (segment (start 110.67218 91.72599) (end 111.00901 92.06282) (width 0.25) (layer F.Cu) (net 2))
 (segment (start 109.29582 91.72599) (end 110.67218 91.72599) (width 0.25) (layer F.Cu) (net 2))
 (segment (start 111.00901 97.50199) (end 110.17 98.341) (width 0.25) (layer F.Cu) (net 2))
 (segment (start 104.14 96.88181) (end 109.29582 91.72599) (width 0.25) (layer F.Cu) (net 2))
 (segment (start 104.14 98.5385) (end 104.14 96.88181) (width 0.25) (layer F.Cu) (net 2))
 (segment (start 115.6605 94.5515) (end 115.10725 95.10475) (width 0.25) (layer F.Cu) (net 2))
 (segment (start 115.6605 93.472) (end 115.6605 94.5515) (width 0.25) (layer F.Cu) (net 2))
 (segment (start 115.10725 95.10475) (end 115.2795 94.9325) (width 0.25) (layer F.Cu) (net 2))
 (segment (start 111.871 98.341) (end 115.10725 95.10475) (width 0.25) (layer F.Cu) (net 2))
 (segment (start 102.9805 97.379) (end 104.14 98.5385) (width 0.25) (layer F.Cu) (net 2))
 (segment (start 99.443 97.379) (end 102.9805 97.379) (width 0.25) (layer F.Cu) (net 2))
 (segment (start 110.17 100.541) (end 110.17 100.523) (width 0.25) (layer F.Cu) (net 3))
 (segment (start 111.6375 100.541) (end 114.681 97.4975) (width 0.25) (layer F.Cu) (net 3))
 (segment (start 110.17 100.541) (end 111.6375 100.541) (width 0.25) (layer F.Cu) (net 3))
 (segment (start 118.1665 97.4975) (end 118.6815 98.0125) (width 0.25) (layer F.Cu) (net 3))
 (segment (start 114.681 97.4975) (end 118.1665 97.4975) (width 0.25) (layer F.Cu) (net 3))
 (segment (start 112.6855 93.1029) (end 112.6855 93.472) (width 0.25) (layer F.Cu) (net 6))
 (segment (start 110.858581 91.275981) (end 112.6855 93.1029) (width 0.25) (layer F.Cu) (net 6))
 (segment (start 106.33402 91.27598) (end 110.858581 91.275981) (width 0.25) (layer F.Cu) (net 6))
 (segment (start 103.884 93.726) (end 106.33402 91.27598) (width 0.25) (layer F.Cu) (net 6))
 (segment (start 99.043 101.579) (end 99.443 101.179) (width 0.25) (layer F.Cu) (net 7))
 (segment (start 96.743 101.579) (end 99.043 101.579) (width 0.25) (layer F.Cu) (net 7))
 (segment (start 96.743 101.579) (end 96.743 95.179) (width 0.25) (layer F.Cu) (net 7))
 (segment (start 98.443 95.179) (end 99.443 96.179) (width 0.25) (layer F.Cu) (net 7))
 (segment (start 96.743 95.179) (end 98.443 95.179) (width 0.25) (layer F.Cu) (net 7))
 (segment (start 106.6145 99.9965) (end 108.27 98.341) (width 0.25) (layer F.Cu) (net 1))
 (segment (start 106.6145 104.775) (end 106.6145 99.9965) (width 0.25) (layer F.Cu) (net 1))
 (segment (start 109.0935 98.9375) (end 109.0935 96.077) (width 0.25) (layer F.Cu) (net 5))
 (segment (start 109.0935 96.077) (end 109.7935 95.377) (width 0.25) (layer F.Cu) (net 5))
 (segment (start 108.27 99.761) (end 109.0935 98.9375) (width 0.25) (layer F.Cu) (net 5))
 (segment (start 108.27 100.541) (end 108.27 99.761) (width 0.25) (layer F.Cu) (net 5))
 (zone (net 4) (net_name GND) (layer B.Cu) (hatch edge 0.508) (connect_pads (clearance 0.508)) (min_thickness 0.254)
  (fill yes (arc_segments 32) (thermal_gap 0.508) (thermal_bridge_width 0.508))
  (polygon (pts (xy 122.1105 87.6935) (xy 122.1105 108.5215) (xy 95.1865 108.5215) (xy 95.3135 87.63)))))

